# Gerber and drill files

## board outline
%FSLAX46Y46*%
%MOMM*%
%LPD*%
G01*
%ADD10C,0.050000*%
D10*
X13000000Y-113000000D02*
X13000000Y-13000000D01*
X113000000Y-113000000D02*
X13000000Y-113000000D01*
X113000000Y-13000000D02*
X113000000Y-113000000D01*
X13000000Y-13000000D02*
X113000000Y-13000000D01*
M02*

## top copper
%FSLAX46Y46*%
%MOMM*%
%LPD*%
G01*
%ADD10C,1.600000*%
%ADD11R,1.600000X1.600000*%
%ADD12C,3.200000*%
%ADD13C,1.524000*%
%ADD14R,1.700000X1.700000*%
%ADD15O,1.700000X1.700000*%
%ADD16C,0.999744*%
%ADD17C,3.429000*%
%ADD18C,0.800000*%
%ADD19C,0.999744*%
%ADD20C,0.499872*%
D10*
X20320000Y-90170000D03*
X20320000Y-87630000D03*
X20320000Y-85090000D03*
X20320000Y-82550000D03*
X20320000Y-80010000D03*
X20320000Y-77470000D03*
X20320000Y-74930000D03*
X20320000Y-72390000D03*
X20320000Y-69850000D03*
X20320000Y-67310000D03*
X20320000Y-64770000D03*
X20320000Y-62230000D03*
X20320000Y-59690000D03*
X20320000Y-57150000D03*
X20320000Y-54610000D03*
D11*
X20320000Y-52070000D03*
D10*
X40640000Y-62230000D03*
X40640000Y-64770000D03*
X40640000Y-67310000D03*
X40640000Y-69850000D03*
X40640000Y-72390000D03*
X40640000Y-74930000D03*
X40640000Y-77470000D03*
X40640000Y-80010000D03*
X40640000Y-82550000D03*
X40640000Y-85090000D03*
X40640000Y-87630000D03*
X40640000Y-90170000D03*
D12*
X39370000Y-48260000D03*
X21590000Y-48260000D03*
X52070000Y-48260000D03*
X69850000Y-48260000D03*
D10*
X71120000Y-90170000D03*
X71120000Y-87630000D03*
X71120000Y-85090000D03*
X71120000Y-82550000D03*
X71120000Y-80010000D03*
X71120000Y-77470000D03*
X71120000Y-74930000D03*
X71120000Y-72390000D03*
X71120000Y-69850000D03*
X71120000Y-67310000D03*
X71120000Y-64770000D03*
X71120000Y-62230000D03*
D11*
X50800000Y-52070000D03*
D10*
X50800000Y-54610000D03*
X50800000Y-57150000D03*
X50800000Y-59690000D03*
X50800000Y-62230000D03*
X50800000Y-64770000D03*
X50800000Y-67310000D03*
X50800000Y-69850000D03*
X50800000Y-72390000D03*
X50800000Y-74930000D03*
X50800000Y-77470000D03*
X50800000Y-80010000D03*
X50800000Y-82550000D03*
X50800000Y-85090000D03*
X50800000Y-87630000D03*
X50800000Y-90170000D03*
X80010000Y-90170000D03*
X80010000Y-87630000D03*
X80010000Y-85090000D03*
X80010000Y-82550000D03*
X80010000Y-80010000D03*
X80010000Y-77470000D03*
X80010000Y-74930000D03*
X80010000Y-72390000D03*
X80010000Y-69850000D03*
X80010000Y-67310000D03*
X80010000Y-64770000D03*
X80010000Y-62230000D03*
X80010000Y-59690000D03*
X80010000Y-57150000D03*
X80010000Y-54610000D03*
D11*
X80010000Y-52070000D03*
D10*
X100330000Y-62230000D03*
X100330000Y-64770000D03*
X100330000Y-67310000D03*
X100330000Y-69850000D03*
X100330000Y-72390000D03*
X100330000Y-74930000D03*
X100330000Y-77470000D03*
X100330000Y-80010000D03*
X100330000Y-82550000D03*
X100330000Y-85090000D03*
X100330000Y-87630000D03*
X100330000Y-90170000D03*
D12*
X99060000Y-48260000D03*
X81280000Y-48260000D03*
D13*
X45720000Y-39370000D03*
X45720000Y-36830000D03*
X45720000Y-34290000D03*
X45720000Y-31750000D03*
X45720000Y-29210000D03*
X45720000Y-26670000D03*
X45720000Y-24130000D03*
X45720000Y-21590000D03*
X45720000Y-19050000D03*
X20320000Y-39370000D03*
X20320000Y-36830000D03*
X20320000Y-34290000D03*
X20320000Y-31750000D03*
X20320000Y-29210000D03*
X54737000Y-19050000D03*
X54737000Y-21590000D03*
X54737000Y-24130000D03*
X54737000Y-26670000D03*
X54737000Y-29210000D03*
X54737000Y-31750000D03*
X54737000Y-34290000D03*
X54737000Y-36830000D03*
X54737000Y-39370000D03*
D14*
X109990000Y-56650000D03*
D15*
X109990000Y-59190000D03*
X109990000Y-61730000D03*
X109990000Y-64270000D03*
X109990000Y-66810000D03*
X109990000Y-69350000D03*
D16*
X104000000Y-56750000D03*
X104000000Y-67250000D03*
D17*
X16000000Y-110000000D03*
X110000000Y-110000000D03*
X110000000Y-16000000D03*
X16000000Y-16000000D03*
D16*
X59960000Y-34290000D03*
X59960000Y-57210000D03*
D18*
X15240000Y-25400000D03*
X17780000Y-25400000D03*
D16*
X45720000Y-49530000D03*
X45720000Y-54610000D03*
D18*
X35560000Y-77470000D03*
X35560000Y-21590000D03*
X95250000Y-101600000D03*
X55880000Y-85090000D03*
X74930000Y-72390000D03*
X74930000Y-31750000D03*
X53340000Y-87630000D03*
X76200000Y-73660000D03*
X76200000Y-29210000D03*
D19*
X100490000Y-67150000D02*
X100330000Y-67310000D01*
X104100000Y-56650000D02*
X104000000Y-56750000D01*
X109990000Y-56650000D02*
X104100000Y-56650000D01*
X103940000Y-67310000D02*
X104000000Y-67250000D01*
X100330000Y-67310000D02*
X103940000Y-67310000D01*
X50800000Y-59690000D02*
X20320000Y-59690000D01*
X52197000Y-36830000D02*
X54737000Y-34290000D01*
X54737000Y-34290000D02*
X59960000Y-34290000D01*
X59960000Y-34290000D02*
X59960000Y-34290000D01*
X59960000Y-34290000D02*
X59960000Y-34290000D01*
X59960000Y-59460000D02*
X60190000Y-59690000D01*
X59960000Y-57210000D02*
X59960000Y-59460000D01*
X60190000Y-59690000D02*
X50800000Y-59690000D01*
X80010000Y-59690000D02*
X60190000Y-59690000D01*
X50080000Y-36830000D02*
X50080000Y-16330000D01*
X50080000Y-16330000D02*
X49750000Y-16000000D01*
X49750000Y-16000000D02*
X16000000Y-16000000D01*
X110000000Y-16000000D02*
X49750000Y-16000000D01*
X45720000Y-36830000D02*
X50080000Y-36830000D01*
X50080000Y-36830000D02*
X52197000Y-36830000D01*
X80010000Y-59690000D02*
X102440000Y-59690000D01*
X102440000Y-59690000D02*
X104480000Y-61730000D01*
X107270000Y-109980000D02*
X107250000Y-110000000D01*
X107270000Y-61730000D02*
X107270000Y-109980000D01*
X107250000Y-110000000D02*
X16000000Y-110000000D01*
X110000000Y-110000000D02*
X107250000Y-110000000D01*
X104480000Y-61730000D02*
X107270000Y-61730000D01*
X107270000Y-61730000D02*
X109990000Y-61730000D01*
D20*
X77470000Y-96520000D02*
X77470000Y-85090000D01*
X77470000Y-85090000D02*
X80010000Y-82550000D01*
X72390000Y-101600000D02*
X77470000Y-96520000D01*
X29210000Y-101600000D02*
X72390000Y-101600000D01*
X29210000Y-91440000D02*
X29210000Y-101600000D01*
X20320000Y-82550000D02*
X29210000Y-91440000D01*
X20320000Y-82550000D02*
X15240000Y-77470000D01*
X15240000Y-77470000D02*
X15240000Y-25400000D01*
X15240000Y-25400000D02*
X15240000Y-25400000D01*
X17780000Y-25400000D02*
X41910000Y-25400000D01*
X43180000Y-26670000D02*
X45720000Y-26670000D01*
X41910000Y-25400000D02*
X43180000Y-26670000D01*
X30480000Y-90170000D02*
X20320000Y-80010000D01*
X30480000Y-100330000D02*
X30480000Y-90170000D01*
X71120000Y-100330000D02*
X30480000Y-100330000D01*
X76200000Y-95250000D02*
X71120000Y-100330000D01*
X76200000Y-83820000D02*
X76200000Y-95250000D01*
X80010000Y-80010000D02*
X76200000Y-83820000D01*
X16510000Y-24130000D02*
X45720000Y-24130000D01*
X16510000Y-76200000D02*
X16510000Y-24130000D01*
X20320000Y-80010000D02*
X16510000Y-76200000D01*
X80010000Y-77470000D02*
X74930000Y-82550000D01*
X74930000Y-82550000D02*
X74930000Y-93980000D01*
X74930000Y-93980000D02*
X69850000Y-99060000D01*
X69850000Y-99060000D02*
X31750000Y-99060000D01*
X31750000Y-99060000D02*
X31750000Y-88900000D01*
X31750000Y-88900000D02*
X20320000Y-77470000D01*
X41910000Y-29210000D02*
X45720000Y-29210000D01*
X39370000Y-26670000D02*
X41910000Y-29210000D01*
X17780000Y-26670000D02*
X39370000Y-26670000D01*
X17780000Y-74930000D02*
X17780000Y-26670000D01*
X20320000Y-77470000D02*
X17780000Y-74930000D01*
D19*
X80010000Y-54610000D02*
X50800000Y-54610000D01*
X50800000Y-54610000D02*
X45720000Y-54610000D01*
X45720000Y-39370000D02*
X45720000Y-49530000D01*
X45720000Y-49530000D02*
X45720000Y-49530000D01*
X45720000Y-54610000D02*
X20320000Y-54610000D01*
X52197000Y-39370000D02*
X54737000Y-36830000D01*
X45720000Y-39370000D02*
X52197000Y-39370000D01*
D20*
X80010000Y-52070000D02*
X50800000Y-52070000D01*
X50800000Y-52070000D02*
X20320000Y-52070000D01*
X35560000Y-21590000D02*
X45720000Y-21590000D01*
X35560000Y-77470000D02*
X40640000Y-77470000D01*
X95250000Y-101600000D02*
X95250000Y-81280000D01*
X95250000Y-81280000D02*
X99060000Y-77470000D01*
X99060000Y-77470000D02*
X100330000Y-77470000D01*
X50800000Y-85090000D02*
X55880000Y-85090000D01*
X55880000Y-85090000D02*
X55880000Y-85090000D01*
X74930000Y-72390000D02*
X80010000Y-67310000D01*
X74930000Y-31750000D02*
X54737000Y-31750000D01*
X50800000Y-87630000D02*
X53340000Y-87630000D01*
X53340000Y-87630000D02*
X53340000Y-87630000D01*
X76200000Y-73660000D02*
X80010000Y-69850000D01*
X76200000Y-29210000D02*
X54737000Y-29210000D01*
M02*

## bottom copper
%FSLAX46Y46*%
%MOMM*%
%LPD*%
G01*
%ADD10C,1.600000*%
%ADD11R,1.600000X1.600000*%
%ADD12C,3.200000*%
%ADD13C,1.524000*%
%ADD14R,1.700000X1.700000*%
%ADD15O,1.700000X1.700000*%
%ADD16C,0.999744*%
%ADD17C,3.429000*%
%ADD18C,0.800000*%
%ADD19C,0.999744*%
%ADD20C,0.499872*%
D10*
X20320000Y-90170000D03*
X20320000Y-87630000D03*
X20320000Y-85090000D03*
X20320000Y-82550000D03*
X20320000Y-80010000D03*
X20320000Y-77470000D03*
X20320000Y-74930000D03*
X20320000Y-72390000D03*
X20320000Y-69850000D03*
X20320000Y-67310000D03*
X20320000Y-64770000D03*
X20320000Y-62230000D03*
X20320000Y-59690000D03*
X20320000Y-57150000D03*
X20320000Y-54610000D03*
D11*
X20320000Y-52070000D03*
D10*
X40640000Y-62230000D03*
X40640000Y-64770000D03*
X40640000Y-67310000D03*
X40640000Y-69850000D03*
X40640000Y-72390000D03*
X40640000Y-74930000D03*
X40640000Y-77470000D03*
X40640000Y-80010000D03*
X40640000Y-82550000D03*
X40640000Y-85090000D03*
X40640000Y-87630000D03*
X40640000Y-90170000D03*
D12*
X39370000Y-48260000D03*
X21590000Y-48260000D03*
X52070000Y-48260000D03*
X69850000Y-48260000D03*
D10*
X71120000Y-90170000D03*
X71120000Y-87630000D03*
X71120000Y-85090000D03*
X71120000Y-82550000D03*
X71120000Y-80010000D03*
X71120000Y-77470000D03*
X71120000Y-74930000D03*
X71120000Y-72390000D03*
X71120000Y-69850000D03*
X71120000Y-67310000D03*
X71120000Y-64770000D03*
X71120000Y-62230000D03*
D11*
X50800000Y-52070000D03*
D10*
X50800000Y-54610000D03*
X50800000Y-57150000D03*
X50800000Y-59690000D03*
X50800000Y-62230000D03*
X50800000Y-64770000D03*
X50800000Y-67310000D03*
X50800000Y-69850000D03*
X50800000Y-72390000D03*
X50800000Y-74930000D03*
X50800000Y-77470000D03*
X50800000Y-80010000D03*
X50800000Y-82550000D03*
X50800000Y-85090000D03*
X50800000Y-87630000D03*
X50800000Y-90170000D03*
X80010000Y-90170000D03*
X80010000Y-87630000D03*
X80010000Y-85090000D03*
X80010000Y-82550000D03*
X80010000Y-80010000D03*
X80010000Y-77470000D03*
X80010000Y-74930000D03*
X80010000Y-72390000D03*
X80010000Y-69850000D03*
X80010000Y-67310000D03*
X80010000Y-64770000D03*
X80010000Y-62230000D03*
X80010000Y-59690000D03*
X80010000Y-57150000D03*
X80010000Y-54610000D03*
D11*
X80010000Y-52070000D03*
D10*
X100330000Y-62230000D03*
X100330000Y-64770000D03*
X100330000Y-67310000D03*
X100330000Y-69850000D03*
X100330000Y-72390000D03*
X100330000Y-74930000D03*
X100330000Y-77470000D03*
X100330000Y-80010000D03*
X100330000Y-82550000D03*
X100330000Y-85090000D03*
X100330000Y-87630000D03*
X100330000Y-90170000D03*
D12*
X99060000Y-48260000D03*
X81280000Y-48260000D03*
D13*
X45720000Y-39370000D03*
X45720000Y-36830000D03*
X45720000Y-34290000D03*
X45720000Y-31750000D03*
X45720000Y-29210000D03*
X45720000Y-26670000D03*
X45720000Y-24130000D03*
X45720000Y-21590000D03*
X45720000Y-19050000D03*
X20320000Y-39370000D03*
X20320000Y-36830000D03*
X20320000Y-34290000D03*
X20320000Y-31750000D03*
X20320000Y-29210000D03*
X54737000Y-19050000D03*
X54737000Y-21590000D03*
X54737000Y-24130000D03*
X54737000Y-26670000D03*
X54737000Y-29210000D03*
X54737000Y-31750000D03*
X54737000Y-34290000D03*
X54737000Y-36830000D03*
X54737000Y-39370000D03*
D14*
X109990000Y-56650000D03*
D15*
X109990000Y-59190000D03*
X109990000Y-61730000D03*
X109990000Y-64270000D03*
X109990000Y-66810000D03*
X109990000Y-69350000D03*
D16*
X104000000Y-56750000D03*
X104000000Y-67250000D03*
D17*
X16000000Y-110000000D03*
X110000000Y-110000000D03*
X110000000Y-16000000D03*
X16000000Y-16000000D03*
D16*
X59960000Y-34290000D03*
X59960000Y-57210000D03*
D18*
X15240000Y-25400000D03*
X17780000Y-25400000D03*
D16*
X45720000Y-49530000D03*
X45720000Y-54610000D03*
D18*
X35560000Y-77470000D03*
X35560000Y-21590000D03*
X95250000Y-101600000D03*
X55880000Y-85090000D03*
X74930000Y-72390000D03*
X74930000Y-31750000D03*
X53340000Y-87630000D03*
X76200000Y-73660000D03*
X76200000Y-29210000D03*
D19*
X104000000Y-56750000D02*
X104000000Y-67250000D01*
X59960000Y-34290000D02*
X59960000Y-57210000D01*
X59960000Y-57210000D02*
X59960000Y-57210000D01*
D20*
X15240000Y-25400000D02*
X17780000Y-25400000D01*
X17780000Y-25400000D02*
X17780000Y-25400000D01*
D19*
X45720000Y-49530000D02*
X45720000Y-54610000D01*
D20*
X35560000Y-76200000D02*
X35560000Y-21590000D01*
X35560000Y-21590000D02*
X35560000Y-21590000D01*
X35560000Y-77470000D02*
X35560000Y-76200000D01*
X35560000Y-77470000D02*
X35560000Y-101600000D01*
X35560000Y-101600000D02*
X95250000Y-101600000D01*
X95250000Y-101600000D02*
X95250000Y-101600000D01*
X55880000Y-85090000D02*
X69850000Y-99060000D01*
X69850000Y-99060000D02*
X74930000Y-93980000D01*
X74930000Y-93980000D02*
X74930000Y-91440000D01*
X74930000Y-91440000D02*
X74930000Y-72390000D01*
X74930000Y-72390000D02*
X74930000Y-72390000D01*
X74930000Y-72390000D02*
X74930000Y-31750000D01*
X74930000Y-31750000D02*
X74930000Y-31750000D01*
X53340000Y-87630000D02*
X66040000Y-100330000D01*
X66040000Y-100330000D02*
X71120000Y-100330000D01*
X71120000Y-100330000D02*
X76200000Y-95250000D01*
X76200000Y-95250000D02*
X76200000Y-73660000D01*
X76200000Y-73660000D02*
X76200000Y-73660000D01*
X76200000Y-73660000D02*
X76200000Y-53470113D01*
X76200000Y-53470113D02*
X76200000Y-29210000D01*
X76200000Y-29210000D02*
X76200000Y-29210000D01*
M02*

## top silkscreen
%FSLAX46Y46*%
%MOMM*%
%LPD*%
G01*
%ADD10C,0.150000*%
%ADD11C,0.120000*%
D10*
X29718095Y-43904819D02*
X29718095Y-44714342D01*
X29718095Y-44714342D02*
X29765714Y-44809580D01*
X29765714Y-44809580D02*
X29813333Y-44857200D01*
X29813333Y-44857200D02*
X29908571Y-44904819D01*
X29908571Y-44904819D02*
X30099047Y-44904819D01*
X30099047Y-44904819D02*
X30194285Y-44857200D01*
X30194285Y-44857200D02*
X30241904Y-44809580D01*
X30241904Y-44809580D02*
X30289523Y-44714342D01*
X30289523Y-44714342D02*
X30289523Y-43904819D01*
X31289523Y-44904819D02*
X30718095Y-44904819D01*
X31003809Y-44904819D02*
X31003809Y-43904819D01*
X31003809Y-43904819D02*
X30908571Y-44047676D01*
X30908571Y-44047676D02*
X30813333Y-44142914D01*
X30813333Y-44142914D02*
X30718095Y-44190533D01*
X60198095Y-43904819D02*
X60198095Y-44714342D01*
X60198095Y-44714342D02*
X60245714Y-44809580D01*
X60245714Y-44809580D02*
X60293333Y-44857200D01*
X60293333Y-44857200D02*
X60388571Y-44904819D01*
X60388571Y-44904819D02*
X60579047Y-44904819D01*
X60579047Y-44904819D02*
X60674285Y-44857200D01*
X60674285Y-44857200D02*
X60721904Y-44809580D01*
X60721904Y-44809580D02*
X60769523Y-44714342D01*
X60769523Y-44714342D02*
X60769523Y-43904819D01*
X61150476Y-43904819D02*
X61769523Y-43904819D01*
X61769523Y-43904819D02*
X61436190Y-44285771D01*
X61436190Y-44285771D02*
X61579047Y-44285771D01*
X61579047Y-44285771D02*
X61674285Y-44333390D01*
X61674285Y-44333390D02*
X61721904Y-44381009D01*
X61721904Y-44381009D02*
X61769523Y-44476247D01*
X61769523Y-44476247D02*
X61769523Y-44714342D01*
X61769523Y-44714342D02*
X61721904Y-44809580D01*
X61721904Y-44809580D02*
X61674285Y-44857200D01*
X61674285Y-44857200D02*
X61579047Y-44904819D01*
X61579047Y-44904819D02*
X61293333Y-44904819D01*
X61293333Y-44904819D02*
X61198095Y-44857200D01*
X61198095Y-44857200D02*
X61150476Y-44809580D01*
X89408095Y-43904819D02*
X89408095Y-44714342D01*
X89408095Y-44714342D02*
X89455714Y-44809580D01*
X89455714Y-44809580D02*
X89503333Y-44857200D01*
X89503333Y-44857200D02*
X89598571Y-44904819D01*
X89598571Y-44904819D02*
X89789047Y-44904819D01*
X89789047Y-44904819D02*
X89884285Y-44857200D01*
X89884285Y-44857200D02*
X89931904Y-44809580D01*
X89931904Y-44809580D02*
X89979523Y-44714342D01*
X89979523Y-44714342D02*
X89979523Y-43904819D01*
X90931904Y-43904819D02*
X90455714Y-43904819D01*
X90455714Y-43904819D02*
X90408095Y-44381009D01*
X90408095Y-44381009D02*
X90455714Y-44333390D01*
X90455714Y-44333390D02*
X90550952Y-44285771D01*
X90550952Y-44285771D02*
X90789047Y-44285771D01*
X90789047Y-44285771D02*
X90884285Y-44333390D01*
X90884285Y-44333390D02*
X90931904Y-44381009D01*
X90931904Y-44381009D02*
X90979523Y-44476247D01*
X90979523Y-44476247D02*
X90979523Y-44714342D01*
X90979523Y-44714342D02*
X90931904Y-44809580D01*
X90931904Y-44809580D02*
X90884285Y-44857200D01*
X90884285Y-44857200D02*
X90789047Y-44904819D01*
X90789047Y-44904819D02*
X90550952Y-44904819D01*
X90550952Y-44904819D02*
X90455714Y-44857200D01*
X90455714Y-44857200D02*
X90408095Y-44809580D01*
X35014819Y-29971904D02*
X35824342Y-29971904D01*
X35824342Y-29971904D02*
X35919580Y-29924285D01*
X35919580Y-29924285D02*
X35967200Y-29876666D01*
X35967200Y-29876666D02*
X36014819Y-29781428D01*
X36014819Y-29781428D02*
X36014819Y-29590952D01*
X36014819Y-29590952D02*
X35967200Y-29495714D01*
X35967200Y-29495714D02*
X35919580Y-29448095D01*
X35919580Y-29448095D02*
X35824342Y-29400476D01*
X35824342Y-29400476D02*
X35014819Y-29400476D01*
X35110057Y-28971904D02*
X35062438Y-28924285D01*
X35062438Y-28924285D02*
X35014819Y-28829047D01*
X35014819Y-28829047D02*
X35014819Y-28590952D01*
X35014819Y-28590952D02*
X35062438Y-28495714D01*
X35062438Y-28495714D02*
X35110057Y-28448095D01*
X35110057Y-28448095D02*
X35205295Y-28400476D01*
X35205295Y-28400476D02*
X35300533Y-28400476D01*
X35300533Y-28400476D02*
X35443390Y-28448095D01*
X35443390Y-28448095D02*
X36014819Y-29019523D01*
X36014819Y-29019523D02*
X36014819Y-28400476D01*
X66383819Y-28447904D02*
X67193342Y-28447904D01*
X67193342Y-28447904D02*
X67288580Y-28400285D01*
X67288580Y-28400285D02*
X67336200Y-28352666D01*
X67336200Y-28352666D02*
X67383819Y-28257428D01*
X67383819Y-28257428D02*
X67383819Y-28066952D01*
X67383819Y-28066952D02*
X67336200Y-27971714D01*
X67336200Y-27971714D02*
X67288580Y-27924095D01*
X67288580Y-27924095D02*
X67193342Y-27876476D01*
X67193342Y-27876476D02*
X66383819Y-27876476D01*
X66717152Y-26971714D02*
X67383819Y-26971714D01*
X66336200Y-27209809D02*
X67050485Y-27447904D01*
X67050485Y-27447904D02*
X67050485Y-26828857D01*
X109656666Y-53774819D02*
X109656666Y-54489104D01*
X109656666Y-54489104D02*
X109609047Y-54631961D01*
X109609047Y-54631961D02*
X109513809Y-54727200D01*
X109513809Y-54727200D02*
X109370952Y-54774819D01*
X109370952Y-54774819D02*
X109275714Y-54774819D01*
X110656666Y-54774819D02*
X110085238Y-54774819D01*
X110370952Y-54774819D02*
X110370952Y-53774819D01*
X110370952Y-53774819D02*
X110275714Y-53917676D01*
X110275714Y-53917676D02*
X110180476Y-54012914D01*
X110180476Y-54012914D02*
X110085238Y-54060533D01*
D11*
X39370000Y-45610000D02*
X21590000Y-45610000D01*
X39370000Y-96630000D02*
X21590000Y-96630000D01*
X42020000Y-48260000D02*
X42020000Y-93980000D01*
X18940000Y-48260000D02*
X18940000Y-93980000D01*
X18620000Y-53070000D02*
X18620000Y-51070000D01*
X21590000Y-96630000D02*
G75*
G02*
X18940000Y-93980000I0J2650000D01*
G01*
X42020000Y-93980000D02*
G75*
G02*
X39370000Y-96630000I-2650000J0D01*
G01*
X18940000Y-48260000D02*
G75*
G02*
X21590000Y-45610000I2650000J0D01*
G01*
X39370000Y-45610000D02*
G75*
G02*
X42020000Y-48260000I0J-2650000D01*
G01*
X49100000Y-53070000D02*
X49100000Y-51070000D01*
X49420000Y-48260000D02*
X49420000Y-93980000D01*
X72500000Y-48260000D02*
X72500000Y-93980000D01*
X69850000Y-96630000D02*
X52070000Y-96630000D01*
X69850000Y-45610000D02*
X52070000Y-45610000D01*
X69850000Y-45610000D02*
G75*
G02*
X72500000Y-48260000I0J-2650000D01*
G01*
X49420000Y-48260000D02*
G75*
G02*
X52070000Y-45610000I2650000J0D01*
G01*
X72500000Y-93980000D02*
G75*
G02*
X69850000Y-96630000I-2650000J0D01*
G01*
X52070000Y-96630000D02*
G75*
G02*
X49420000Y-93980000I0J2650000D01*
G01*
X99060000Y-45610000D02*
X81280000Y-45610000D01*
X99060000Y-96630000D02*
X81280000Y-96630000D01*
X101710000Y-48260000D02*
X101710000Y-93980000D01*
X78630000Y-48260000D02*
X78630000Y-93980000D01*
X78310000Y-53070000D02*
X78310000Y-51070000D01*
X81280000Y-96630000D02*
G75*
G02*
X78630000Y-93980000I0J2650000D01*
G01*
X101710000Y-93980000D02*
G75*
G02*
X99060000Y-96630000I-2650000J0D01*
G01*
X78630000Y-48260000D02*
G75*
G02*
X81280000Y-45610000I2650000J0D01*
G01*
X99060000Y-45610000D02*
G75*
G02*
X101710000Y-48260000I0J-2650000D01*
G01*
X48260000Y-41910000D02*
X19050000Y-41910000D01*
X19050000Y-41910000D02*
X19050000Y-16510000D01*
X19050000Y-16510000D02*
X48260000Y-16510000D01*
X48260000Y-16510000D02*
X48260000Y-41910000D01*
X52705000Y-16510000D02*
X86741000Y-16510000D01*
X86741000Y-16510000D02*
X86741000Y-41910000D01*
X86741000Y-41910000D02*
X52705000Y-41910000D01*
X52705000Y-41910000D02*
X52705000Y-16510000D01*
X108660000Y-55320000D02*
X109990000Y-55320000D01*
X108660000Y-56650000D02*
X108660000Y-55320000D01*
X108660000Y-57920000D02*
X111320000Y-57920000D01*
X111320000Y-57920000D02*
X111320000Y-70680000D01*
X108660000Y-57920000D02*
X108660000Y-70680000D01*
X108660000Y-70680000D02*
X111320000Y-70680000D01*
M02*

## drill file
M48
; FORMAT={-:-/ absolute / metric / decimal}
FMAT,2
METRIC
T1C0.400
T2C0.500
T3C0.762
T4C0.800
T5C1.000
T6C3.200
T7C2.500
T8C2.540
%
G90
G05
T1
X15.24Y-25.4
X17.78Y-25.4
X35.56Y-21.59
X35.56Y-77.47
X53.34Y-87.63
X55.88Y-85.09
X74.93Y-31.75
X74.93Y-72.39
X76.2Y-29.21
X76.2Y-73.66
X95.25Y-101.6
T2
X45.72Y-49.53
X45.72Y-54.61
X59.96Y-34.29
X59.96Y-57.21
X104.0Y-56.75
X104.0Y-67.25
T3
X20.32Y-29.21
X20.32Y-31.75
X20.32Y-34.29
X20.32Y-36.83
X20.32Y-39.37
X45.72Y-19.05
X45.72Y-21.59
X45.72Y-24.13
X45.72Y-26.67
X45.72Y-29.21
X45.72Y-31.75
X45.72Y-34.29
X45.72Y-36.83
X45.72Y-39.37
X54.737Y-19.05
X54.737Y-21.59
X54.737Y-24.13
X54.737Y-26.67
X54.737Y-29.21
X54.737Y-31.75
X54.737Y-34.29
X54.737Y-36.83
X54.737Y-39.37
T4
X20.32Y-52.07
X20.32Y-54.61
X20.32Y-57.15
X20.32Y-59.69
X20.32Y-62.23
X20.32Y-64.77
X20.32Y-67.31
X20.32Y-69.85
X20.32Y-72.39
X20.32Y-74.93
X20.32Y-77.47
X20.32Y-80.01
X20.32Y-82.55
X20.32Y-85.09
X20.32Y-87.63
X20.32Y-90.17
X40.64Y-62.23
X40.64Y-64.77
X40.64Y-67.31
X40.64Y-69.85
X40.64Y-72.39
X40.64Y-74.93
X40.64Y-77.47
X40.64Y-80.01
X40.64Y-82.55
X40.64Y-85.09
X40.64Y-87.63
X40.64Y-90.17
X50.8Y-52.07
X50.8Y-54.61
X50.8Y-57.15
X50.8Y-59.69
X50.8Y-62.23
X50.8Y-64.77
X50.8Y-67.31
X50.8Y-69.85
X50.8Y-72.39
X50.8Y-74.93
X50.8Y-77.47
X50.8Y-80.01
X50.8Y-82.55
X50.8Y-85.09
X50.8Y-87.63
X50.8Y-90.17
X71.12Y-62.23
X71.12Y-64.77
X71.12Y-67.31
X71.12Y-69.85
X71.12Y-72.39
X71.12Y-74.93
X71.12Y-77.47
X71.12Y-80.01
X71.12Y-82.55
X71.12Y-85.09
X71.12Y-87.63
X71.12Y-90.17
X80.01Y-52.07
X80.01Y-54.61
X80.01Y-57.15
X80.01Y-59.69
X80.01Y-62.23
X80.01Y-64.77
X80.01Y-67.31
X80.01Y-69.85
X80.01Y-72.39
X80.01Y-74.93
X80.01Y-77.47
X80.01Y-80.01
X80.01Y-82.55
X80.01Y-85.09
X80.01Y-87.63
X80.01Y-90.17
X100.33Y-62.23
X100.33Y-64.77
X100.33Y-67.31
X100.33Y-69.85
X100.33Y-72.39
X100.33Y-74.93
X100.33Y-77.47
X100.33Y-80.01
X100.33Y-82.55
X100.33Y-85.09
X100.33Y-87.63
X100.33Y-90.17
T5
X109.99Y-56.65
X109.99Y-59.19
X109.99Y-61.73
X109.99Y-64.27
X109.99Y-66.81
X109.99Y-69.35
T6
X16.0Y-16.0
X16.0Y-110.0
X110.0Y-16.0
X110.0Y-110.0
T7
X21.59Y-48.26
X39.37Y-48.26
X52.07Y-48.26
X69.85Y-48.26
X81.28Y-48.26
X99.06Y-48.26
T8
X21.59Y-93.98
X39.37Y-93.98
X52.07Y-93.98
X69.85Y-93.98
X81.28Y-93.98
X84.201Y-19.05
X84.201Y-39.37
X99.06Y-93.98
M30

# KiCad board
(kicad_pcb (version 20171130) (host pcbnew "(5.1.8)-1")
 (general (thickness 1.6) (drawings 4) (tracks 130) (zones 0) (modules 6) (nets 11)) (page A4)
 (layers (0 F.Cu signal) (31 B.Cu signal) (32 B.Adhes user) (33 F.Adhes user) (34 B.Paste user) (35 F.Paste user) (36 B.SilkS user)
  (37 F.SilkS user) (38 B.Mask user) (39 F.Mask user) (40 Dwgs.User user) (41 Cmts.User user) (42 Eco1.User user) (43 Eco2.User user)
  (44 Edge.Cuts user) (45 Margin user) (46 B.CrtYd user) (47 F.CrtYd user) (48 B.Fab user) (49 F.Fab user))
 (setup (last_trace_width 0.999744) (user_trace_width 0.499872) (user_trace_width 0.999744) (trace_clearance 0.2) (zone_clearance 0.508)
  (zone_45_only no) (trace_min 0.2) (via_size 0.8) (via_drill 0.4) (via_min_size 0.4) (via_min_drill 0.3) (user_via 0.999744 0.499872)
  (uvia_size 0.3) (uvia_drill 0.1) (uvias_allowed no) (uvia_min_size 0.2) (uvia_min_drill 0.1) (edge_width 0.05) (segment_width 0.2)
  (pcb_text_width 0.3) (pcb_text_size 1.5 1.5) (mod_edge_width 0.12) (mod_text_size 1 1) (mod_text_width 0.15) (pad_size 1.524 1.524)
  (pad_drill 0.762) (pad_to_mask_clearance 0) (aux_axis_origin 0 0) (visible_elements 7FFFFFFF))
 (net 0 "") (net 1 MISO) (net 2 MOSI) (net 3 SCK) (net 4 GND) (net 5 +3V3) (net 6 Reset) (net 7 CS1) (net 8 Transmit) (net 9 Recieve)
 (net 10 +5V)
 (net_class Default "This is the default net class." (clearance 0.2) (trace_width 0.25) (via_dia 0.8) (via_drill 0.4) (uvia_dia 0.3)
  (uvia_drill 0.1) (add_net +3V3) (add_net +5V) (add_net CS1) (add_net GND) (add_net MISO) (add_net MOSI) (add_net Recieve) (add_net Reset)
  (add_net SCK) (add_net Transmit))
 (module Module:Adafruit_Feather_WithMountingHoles (layer F.Cu) (at 20.32 52.07)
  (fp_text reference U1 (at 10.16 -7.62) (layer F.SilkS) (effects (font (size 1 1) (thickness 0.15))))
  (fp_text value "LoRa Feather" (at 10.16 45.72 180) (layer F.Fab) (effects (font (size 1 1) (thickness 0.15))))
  (fp_line (start 19.05 -6.46) (end 1.27 -6.46) (layer F.SilkS) (width 0.12))
  (fp_line (start 19.05 44.56) (end 1.27 44.56) (layer F.SilkS) (width 0.12))
  (fp_line (start 21.7 -3.81) (end 21.7 41.91) (layer F.SilkS) (width 0.12))
  (fp_line (start -1.38 -3.81) (end -1.38 41.91) (layer F.SilkS) (width 0.12))
  (fp_line (start -1.7 1) (end -1.7 -1) (layer F.SilkS) (width 0.12))
  (fp_arc (start 1.27 41.91) (end -1.38 41.91) (angle -90) (layer F.SilkS) (width 0.12))
  (fp_arc (start 19.05 41.91) (end 19.05 44.56) (angle -90) (layer F.SilkS) (width 0.12))
  (fp_arc (start 1.27 -3.81) (end 1.27 -6.46) (angle -90) (layer F.SilkS) (width 0.12))
  (fp_arc (start 19.05 -3.81) (end 21.7 -3.81) (angle -90) (layer F.SilkS) (width 0.12))
  (pad 16 thru_hole circle (at 0 38.1 180) (size 1.6 1.6) (drill 0.8) (layers *.Cu *.Mask))
  (pad 15 thru_hole circle (at 0 35.56 180) (size 1.6 1.6) (drill 0.8) (layers *.Cu *.Mask))
  (pad 14 thru_hole circle (at 0 33.02 180) (size 1.6 1.6) (drill 0.8) (layers *.Cu *.Mask))
  (pad 13 thru_hole circle (at 0 30.48 180) (size 1.6 1.6) (drill 0.8) (layers *.Cu *.Mask) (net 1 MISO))
  (pad 12 thru_hole circle (at 0 27.94 180) (size 1.6 1.6) (drill 0.8) (layers *.Cu *.Mask) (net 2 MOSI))
  (pad 11 thru_hole circle (at 0 25.4 180) (size 1.6 1.6) (drill 0.8) (layers *.Cu *.Mask) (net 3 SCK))
  (pad 10 thru_hole circle (at 0 22.86 180) (size 1.6 1.6) (drill 0.8) (layers *.Cu *.Mask))
  (pad 9 thru_hole circle (at 0 20.32 180) (size 1.6 1.6) (drill 0.8) (layers *.Cu *.Mask))
  (pad 8 thru_hole circle (at 0 17.78 180) (size 1.6 1.6) (drill 0.8) (layers *.Cu *.Mask))
  (pad 7 thru_hole circle (at 0 15.24 180) (size 1.6 1.6) (drill 0.8) (layers *.Cu *.Mask))
  (pad 6 thru_hole circle (at 0 12.7 180) (size 1.6 1.6) (drill 0.8) (layers *.Cu *.Mask))
  (pad 5 thru_hole circle (at 0 10.16 180) (size 1.6 1.6) (drill 0.8) (layers *.Cu *.Mask))
  (pad 4 thru_hole circle (at 0 7.62 180) (size 1.6 1.6) (drill 0.8) (layers *.Cu *.Mask) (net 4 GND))
  (pad 3 thru_hole circle (at 0 5.08 180) (size 1.6 1.6) (drill 0.8) (layers *.Cu *.Mask))
  (pad 2 thru_hole circle (at 0 2.54 180) (size 1.6 1.6) (drill 0.8) (layers *.Cu *.Mask) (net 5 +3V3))
  (pad 1 thru_hole rect (at 0 0 180) (size 1.6 1.6) (drill 0.8) (layers *.Cu *.Mask) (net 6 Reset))
  (pad 28 thru_hole circle (at 20.32 10.16 180) (size 1.6 1.6) (drill 0.8) (layers *.Cu *.Mask))
  (pad 27 thru_hole circle (at 20.32 12.7 180) (size 1.6 1.6) (drill 0.8) (layers *.Cu *.Mask))
  (pad 26 thru_hole circle (at 20.32 15.24 180) (size 1.6 1.6) (drill 0.8) (layers *.Cu *.Mask))
  (pad 25 thru_hole circle (at 20.32 17.78 180) (size 1.6 1.6) (drill 0.8) (layers *.Cu *.Mask))
  (pad 24 thru_hole circle (at 20.32 20.32 180) (size 1.6 1.6) (drill 0.8) (layers *.Cu *.Mask))
  (pad 23 thru_hole circle (at 20.32 22.86 180) (size 1.6 1.6) (drill 0.8) (layers *.Cu *.Mask))
  (pad 22 thru_hole circle (at 20.32 25.4 180) (size 1.6 1.6) (drill 0.8) (layers *.Cu *.Mask) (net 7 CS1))
  (pad 21 thru_hole circle (at 20.32 27.94 180) (size 1.6 1.6) (drill 0.8) (layers *.Cu *.Mask))
  (pad 20 thru_hole circle (at 20.32 30.48 180) (size 1.6 1.6) (drill 0.8) (layers *.Cu *.Mask))
  (pad 19 thru_hole circle (at 20.32 33.02 180) (size 1.6 1.6) (drill 0.8) (layers *.Cu *.Mask))
  (pad 18 thru_hole circle (at 20.32 35.56 180) (size 1.6 1.6) (drill 0.8) (layers *.Cu *.Mask))
  (pad 17 thru_hole circle (at 20.32 38.1 180) (size 1.6 1.6) (drill 0.8) (layers *.Cu *.Mask))
  (pad "" np_thru_hole circle (at 19.05 -3.81 270) (size 3.2 3.2) (drill 2.5) (layers *.Cu *.Mask))
  (pad "" np_thru_hole circle (at 19.05 41.91 270) (size 2.54 2.54) (drill 2.54) (layers *.Cu *.Mask))
  (pad "" np_thru_hole circle (at 1.27 -3.81 270) (size 3.2 3.2) (drill 2.5) (layers *.Cu *.Mask))
  (pad "" np_thru_hole circle (at 1.27 41.91 270) (size 2.54 2.54) (drill 2.54) (layers *.Cu *.Mask)))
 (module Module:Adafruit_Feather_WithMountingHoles (layer F.Cu) (at 50.8 52.07)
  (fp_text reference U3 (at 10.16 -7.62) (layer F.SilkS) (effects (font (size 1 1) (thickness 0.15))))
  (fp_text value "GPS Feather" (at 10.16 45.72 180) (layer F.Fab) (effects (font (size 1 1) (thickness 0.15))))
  (fp_line (start -1.7 1) (end -1.7 -1) (layer F.SilkS) (width 0.12))
  (fp_line (start -1.38 -3.81) (end -1.38 41.91) (layer F.SilkS) (width 0.12))
  (fp_line (start 21.7 -3.81) (end 21.7 41.91) (layer F.SilkS) (width 0.12))
  (fp_line (start 19.05 44.56) (end 1.27 44.56) (layer F.SilkS) (width 0.12))
  (fp_line (start 19.05 -6.46) (end 1.27 -6.46) (layer F.SilkS) (width 0.12))
  (fp_arc (start 19.05 -3.81) (end 21.7 -3.81) (angle -90) (layer F.SilkS) (width 0.12))
  (fp_arc (start 1.27 -3.81) (end 1.27 -6.46) (angle -90) (layer F.SilkS) (width 0.12))
  (fp_arc (start 19.05 41.91) (end 19.05 44.56) (angle -90) (layer F.SilkS) (width 0.12))
  (fp_arc (start 1.27 41.91) (end -1.38 41.91) (angle -90) (layer F.SilkS) (width 0.12))
  (pad "" np_thru_hole circle (at 1.27 41.91 270) (size 2.54 2.54) (drill 2.54) (layers *.Cu *.Mask))
  (pad "" np_thru_hole circle (at 1.27 -3.81 270) (size 3.2 3.2) (drill 2.5) (layers *.Cu *.Mask))
  (pad "" np_thru_hole circle (at 19.05 41.91 270) (size 2.54 2.54) (drill 2.54) (layers *.Cu *.Mask))
  (pad "" np_thru_hole circle (at 19.05 -3.81 270) (size 3.2 3.2) (drill 2.5) (layers *.Cu *.Mask))
  (pad 17 thru_hole circle (at 20.32 38.1 180) (size 1.6 1.6) (drill 0.8) (layers *.Cu *.Mask))
  (pad 18 thru_hole circle (at 20.32 35.56 180) (size 1.6 1.6) (drill 0.8) (layers *.Cu *.Mask))
  (pad 19 thru_hole circle (at 20.32 33.02 180) (size 1.6 1.6) (drill 0.8) (layers *.Cu *.Mask))
  (pad 20 thru_hole circle (at 20.32 30.48 180) (size 1.6 1.6) (drill 0.8) (layers *.Cu *.Mask))
  (pad 21 thru_hole circle (at 20.32 27.94 180) (size 1.6 1.6) (drill 0.8) (layers *.Cu *.Mask))
  (pad 22 thru_hole circle (at 20.32 25.4 180) (size 1.6 1.6) (drill 0.8) (layers *.Cu *.Mask))
  (pad 23 thru_hole circle (at 20.32 22.86 180) (size 1.6 1.6) (drill 0.8) (layers *.Cu *.Mask))
  (pad 24 thru_hole circle (at 20.32 20.32 180) (size 1.6 1.6) (drill 0.8) (layers *.Cu *.Mask))
  (pad 25 thru_hole circle (at 20.32 17.78 180) (size 1.6 1.6) (drill 0.8) (layers *.Cu *.Mask))
  (pad 26 thru_hole circle (at 20.32 15.24 180) (size 1.6 1.6) (drill 0.8) (layers *.Cu *.Mask))
  (pad 27 thru_hole circle (at 20.32 12.7 180) (size 1.6 1.6) (drill 0.8) (layers *.Cu *.Mask))
  (pad 28 thru_hole circle (at 20.32 10.16 180) (size 1.6 1.6) (drill 0.8) (layers *.Cu *.Mask))
  (pad 1 thru_hole rect (at 0 0 180) (size 1.6 1.6) (drill 0.8) (layers *.Cu *.Mask) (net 6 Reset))
  (pad 2 thru_hole circle (at 0 2.54 180) (size 1.6 1.6) (drill 0.8) (layers *.Cu *.Mask) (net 5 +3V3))
  (pad 3 thru_hole circle (at 0 5.08 180) (size 1.6 1.6) (drill 0.8) (layers *.Cu *.Mask))
  (pad 4 thru_hole circle (at 0 7.62 180) (size 1.6 1.6) (drill 0.8) (layers *.Cu *.Mask) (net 4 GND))
  (pad 5 thru_hole circle (at 0 10.16 180) (size 1.6 1.6) (drill 0.8) (layers *.Cu *.Mask))
  (pad 6 thru_hole circle (at 0 12.7 180) (size 1.6 1.6) (drill 0.8) (layers *.Cu *.Mask))
  (pad 7 thru_hole circle (at 0 15.24 180) (size 1.6 1.6) (drill 0.8) (layers *.Cu *.Mask))
  (pad 8 thru_hole circle (at 0 17.78 180) (size 1.6 1.6) (drill 0.8) (layers *.Cu *.Mask))
  (pad 9 thru_hole circle (at 0 20.32 180) (size 1.6 1.6) (drill 0.8) (layers *.Cu *.Mask))
  (pad 10 thru_hole circle (at 0 22.86 180) (size 1.6 1.6) (drill 0.8) (layers *.Cu *.Mask))
  (pad 11 thru_hole circle (at 0 25.4 180) (size 1.6 1.6) (drill 0.8) (layers *.Cu *.Mask))
  (pad 12 thru_hole circle (at 0 27.94 180) (size 1.6 1.6) (drill 0.8) (layers *.Cu *.Mask))
  (pad 13 thru_hole circle (at 0 30.48 180) (size 1.6 1.6) (drill 0.8) (layers *.Cu *.Mask))
  (pad 14 thru_hole circle (at 0 33.02 180) (size 1.6 1.6) (drill 0.8) (layers *.Cu *.Mask) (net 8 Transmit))
  (pad 15 thru_hole circle (at 0 35.56 180) (size 1.6 1.6) (drill 0.8) (layers *.Cu *.Mask) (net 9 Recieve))
  (pad 16 thru_hole circle (at 0 38.1 180) (size 1.6 1.6) (drill 0.8) (layers *.Cu *.Mask)))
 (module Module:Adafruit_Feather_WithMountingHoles (layer F.Cu) (at 80.01 52.07)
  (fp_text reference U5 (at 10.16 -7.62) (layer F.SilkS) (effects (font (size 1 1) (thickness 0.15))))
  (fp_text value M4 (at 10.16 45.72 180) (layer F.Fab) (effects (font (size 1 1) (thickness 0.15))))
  (fp_line (start 19.05 -6.46) (end 1.27 -6.46) (layer F.SilkS) (width 0.12))
  (fp_line (start 19.05 44.56) (end 1.27 44.56) (layer F.SilkS) (width 0.12))
  (fp_line (start 21.7 -3.81) (end 21.7 41.91) (layer F.SilkS) (width 0.12))
  (fp_line (start -1.38 -3.81) (end -1.38 41.91) (layer F.SilkS) (width 0.12))
  (fp_line (start -1.7 1) (end -1.7 -1) (layer F.SilkS) (width 0.12))
  (fp_arc (start 1.27 41.91) (end -1.38 41.91) (angle -90) (layer F.SilkS) (width 0.12))
  (fp_arc (start 19.05 41.91) (end 19.05 44.56) (angle -90) (layer F.SilkS) (width 0.12))
  (fp_arc (start 1.27 -3.81) (end 1.27 -6.46) (angle -90) (layer F.SilkS) (width 0.12))
  (fp_arc (start 19.05 -3.81) (end 21.7 -3.81) (angle -90) (layer F.SilkS) (width 0.12))
  (pad 16 thru_hole circle (at 0 38.1 180) (size 1.6 1.6) (drill 0.8) (layers *.Cu *.Mask))
  (pad 15 thru_hole circle (at 0 35.56 180) (size 1.6 1.6) (drill 0.8) (layers *.Cu *.Mask))
  (pad 14 thru_hole circle (at 0 33.02 180) (size 1.6 1.6) (drill 0.8) (layers *.Cu *.Mask))
  (pad 13 thru_hole circle (at 0 30.48 180) (size 1.6 1.6) (drill 0.8) (layers *.Cu *.Mask) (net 1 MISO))
  (pad 12 thru_hole circle (at 0 27.94 180) (size 1.6 1.6) (drill 0.8) (layers *.Cu *.Mask) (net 2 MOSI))
  (pad 11 thru_hole circle (at 0 25.4 180) (size 1.6 1.6) (drill 0.8) (layers *.Cu *.Mask) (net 3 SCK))
  (pad 10 thru_hole circle (at 0 22.86 180) (size 1.6 1.6) (drill 0.8) (layers *.Cu *.Mask))
  (pad 9 thru_hole circle (at 0 20.32 180) (size 1.6 1.6) (drill 0.8) (layers *.Cu *.Mask))
  (pad 8 thru_hole circle (at 0 17.78 180) (size 1.6 1.6) (drill 0.8) (layers *.Cu *.Mask) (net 9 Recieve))
  (pad 7 thru_hole circle (at 0 15.24 180) (size 1.6 1.6) (drill 0.8) (layers *.Cu *.Mask) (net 8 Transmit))
  (pad 6 thru_hole circle (at 0 12.7 180) (size 1.6 1.6) (drill 0.8) (layers *.Cu *.Mask))
  (pad 5 thru_hole circle (at 0 10.16 180) (size 1.6 1.6) (drill 0.8) (layers *.Cu *.Mask))
  (pad 4 thru_hole circle (at 0 7.62 180) (size 1.6 1.6) (drill 0.8) (layers *.Cu *.Mask) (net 4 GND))
  (pad 3 thru_hole circle (at 0 5.08 180) (size 1.6 1.6) (drill 0.8) (layers *.Cu *.Mask))
  (pad 2 thru_hole circle (at 0 2.54 180) (size 1.6 1.6) (drill 0.8) (layers *.Cu *.Mask) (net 5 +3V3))
  (pad 1 thru_hole rect (at 0 0 180) (size 1.6 1.6) (drill 0.8) (layers *.Cu *.Mask) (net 6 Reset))
  (pad 28 thru_hole circle (at 20.32 10.16 180) (size 1.6 1.6) (drill 0.8) (layers *.Cu *.Mask))
  (pad 27 thru_hole circle (at 20.32 12.7 180) (size 1.6 1.6) (drill 0.8) (layers *.Cu *.Mask))
  (pad 26 thru_hole circle (at 20.32 15.24 180) (size 1.6 1.6) (drill 0.8) (layers *.Cu *.Mask) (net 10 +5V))
  (pad 25 thru_hole circle (at 20.32 17.78 180) (size 1.6 1.6) (drill 0.8) (layers *.Cu *.Mask))
  (pad 24 thru_hole circle (at 20.32 20.32 180) (size 1.6 1.6) (drill 0.8) (layers *.Cu *.Mask))
  (pad 23 thru_hole circle (at 20.32 22.86 180) (size 1.6 1.6) (drill 0.8) (layers *.Cu *.Mask))
  (pad 22 thru_hole circle (at 20.32 25.4 180) (size 1.6 1.6) (drill 0.8) (layers *.Cu *.Mask) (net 7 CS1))
  (pad 21 thru_hole circle (at 20.32 27.94 180) (size 1.6 1.6) (drill 0.8) (layers *.Cu *.Mask))
  (pad 20 thru_hole circle (at 20.32 30.48 180) (size 1.6 1.6) (drill 0.8) (layers *.Cu *.Mask))
  (pad 19 thru_hole circle (at 20.32 33.02 180) (size 1.6 1.6) (drill 0.8) (layers *.Cu *.Mask))
  (pad 18 thru_hole circle (at 20.32 35.56 180) (size 1.6 1.6) (drill 0.8) (layers *.Cu *.Mask))
  (pad 17 thru_hole circle (at 20.32 38.1 180) (size 1.6 1.6) (drill 0.8) (layers *.Cu *.Mask))
  (pad "" np_thru_hole circle (at 19.05 -3.81 270) (size 3.2 3.2) (drill 2.5) (layers *.Cu *.Mask))
  (pad "" np_thru_hole circle (at 19.05 41.91 270) (size 2.54 2.54) (drill 2.54) (layers *.Cu *.Mask))
  (pad "" np_thru_hole circle (at 1.27 -3.81 270) (size 3.2 3.2) (drill 2.5) (layers *.Cu *.Mask))
  (pad "" np_thru_hole circle (at 1.27 41.91 270) (size 2.54 2.54) (drill 2.54) (layers *.Cu *.Mask)))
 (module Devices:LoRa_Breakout (layer F.Cu) (at 48.26 41.91 90)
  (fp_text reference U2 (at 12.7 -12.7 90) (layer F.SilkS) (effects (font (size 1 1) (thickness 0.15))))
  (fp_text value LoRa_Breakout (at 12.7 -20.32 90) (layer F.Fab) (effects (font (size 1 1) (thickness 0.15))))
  (fp_line (start 0 0) (end 0 -29.21) (layer F.SilkS) (width 0.12))
  (fp_line (start 0 -29.21) (end 25.4 -29.21) (layer F.SilkS) (width 0.12))
  (fp_line (start 25.4 -29.21) (end 25.4 0) (layer F.SilkS) (width 0.12))
  (fp_line (start 25.4 0) (end 0 0) (layer F.SilkS) (width 0.12))
  (pad 1 thru_hole circle (at 2.54 -2.54 90) (size 1.524 1.524) (drill 0.762) (layers *.Cu *.Mask) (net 5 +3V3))
  (pad 2 thru_hole circle (at 5.08 -2.54 90) (size 1.524 1.524) (drill 0.762) (layers *.Cu *.Mask) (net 4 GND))
  (pad 3 thru_hole circle (at 7.62 -2.54 90) (size 1.524 1.524) (drill 0.762) (layers *.Cu *.Mask))
  (pad 4 thru_hole circle (at 10.16 -2.54 90) (size 1.524 1.524) (drill 0.762) (layers *.Cu *.Mask))
  (pad 5 thru_hole circle (at 12.7 -2.54 90) (size 1.524 1.524) (drill 0.762) (layers *.Cu *.Mask) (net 3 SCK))
  (pad 6 thru_hole circle (at 15.24 -2.54 90) (size 1.524 1.524) (drill 0.762) (layers *.Cu *.Mask) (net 1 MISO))
  (pad 7 thru_hole circle (at 17.78 -2.54 90) (size 1.524 1.524) (drill 0.762) (layers *.Cu *.Mask) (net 2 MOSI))
  (pad 8 thru_hole circle (at 20.32 -2.54 90) (size 1.524 1.524) (drill 0.762) (layers *.Cu *.Mask) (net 7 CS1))
  (pad 9 thru_hole circle (at 22.86 -2.54 90) (size 1.524 1.524) (drill 0.762) (layers *.Cu *.Mask))
  (pad 10 thru_hole circle (at 2.54 -27.94 90) (size 1.524 1.524) (drill 0.762) (layers *.Cu *.Mask))
  (pad 11 thru_hole circle (at 5.08 -27.94 90) (size 1.524 1.524) (drill 0.762) (layers *.Cu *.Mask))
  (pad 12 thru_hole circle (at 7.62 -27.94 90) (size 1.524 1.524) (drill 0.762) (layers *.Cu *.Mask))
  (pad 13 thru_hole circle (at 10.16 -27.94 90) (size 1.524 1.524) (drill 0.762) (layers *.Cu *.Mask))
  (pad 14 thru_hole circle (at 12.7 -27.94 90) (size 1.524 1.524) (drill 0.762) (layers *.Cu *.Mask)))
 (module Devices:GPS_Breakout (layer F.Cu) (at 52.705 16.51 270)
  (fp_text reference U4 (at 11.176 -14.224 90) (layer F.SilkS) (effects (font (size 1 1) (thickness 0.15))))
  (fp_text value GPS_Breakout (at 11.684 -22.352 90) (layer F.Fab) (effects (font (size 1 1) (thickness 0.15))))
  (fp_line (start 0 0) (end 0 -34.036) (layer F.SilkS) (width 0.12))
  (fp_line (start 0 -34.036) (end 25.4 -34.036) (layer F.SilkS) (width 0.12))
  (fp_line (start 25.4 -34.036) (end 25.4 0) (layer F.SilkS) (width 0.12))
  (fp_line (start 25.4 0) (end 0 0) (layer F.SilkS) (width 0.12))
  (pad 1 thru_hole circle (at 2.54 -2.032 270) (size 1.524 1.524) (drill 0.762) (layers *.Cu *.Mask))
  (pad 2 thru_hole circle (at 5.08 -2.032 270) (size 1.524 1.524) (drill 0.762) (layers *.Cu *.Mask))
  (pad 3 thru_hole circle (at 7.62 -2.032 270) (size 1.524 1.524) (drill 0.762) (layers *.Cu *.Mask))
  (pad 4 thru_hole circle (at 10.16 -2.032 270) (size 1.524 1.524) (drill 0.762) (layers *.Cu *.Mask))
  (pad 5 thru_hole circle (at 12.7 -2.032 270) (size 1.524 1.524) (drill 0.762) (layers *.Cu *.Mask) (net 9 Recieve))
  (pad 6 thru_hole circle (at 15.24 -2.032 270) (size 1.524 1.524) (drill 0.762) (layers *.Cu *.Mask) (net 8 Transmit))
  (pad 7 thru_hole circle (at 17.78 -2.032 270) (size 1.524 1.524) (drill 0.762) (layers *.Cu *.Mask) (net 4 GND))
  (pad 8 thru_hole circle (at 20.32 -2.032 270) (size 1.524 1.524) (drill 0.762) (layers *.Cu *.Mask) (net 5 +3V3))
  (pad 9 thru_hole circle (at 22.86 -2.032 270) (size 1.524 1.524) (drill 0.762) (layers *.Cu *.Mask))
  (pad "" np_thru_hole circle (at 2.54 -31.496 270) (size 2.54 2.54) (drill 2.54) (layers *.Cu *.Mask))
  (pad "" np_thru_hole circle (at 22.86 -31.496 270) (size 2.54 2.54) (drill 2.54) (layers *.Cu *.Mask)))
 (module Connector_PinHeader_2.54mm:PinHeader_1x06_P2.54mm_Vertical (layer F.Cu) (at 109.99 56.65)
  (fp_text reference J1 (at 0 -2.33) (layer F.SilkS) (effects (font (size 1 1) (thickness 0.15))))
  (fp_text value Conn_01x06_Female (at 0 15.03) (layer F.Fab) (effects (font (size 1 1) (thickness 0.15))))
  (fp_line (start -1.33 -1.33) (end 0 -1.33) (layer F.SilkS) (width 0.12))
  (fp_line (start -1.33 0) (end -1.33 -1.33) (layer F.SilkS) (width 0.12))
  (fp_line (start -1.33 1.27) (end 1.33 1.27) (layer F.SilkS) (width 0.12))
  (fp_line (start 1.33 1.27) (end 1.33 14.03) (layer F.SilkS) (width 0.12))
  (fp_line (start -1.33 1.27) (end -1.33 14.03) (layer F.SilkS) (width 0.12))
  (fp_line (start -1.33 14.03) (end 1.33 14.03) (layer F.SilkS) (width 0.12))
  (pad 1 thru_hole rect (at 0 0) (size 1.7 1.7) (drill 1) (layers *.Cu *.Mask) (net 10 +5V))
  (pad 2 thru_hole oval (at 0 2.54) (size 1.7 1.7) (drill 1) (layers *.Cu *.Mask))
  (pad 3 thru_hole oval (at 0 5.08) (size 1.7 1.7) (drill 1) (layers *.Cu *.Mask) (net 4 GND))
  (pad 4 thru_hole oval (at 0 7.62) (size 1.7 1.7) (drill 1) (layers *.Cu *.Mask))
  (pad 5 thru_hole oval (at 0 10.16) (size 1.7 1.7) (drill 1) (layers *.Cu *.Mask))
  (pad 6 thru_hole oval (at 0 12.7) (size 1.7 1.7) (drill 1) (layers *.Cu *.Mask)))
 (gr_line (start 13 113) (end 13 13) (layer Edge.Cuts) (width 0.05))
 (gr_line (start 113 113) (end 13 113) (layer Edge.Cuts) (width 0.05))
 (gr_line (start 113 13) (end 113 113) (layer Edge.Cuts) (width 0.05))
 (gr_line (start 13 13) (end 113 13) (layer Edge.Cuts) (width 0.05))
 (via (at 104 56.75) (size 0.999744) (drill 0.499872) (layers F.Cu B.Cu) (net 10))
 (segment (start 104 56.75) (end 104 67.25) (width 0.999744) (layer B.Cu) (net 10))
 (via (at 104 67.25) (size 0.999744) (drill 0.499872) (layers F.Cu B.Cu) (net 10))
 (segment (start 100.49 67.15) (end 100.33 67.31) (width 0.999744) (layer F.Cu) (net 10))
 (segment (start 104.1 56.65) (end 104 56.75) (width 0.999744) (layer F.Cu) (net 10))
 (segment (start 109.99 56.65) (end 104.1 56.65) (width 0.999744) (layer F.Cu) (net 10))
 (segment (start 103.94 67.31) (end 104 67.25) (width 0.999744) (layer F.Cu) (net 10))
 (segment (start 100.33 67.31) (end 103.94 67.31) (width 0.999744) (layer F.Cu) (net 10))
 (via (at 16 110) (size 3.429) (drill 3.2004) (layers F.Cu B.Cu) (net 4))
 (segment (start 50.8 59.69) (end 20.32 59.69) (width 0.999744) (layer F.Cu) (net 4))
 (segment (start 52.197 36.83) (end 54.737 34.29) (width 0.999744) (layer F.Cu) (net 4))
 (via (at 110 110) (size 3.429) (drill 3.2004) (layers F.Cu B.Cu) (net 4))
 (via (at 110 16) (size 3.429) (drill 3.2004) (layers F.Cu B.Cu) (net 4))
 (via (at 16 16) (size 3.429) (drill 3.2004) (layers F.Cu B.Cu) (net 4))
 (segment (start 54.737 34.29) (end 59.96 34.29) (width 0.999744) (layer F.Cu) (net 4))
 (segment (start 59.96 34.29) (end 59.96 34.29) (width 0.999744) (layer F.Cu) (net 4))
 (segment (start 59.96 34.29) (end 59.96 34.29) (width 0.999744) (layer F.Cu) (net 4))
 (via (at 59.96 34.29) (size 0.999744) (drill 0.499872) (layers F.Cu B.Cu) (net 4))
 (segment (start 59.96 34.29) (end 59.96 57.21) (width 0.999744) (layer B.Cu) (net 4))
 (segment (start 59.96 57.21) (end 59.96 57.21) (width 0.999744) (layer B.Cu) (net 4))
 (via (at 59.96 57.21) (size 0.999744) (drill 0.499872) (layers F.Cu B.Cu) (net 4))
 (segment (start 59.96 59.46) (end 60.19 59.69) (width 0.999744) (layer F.Cu) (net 4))
 (segment (start 59.96 57.21) (end 59.96 59.46) (width 0.999744) (layer F.Cu) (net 4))
 (segment (start 60.19 59.69) (end 50.8 59.69) (width 0.999744) (layer F.Cu) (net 4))
 (segment (start 80.01 59.69) (end 60.19 59.69) (width 0.999744) (layer F.Cu) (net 4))
 (segment (start 50.08 36.83) (end 50.08 16.33) (width 0.999744) (layer F.Cu) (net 4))
 (segment (start 50.08 16.33) (end 49.75 16) (width 0.999744) (layer F.Cu) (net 4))
 (segment (start 49.75 16) (end 16 16) (width 0.999744) (layer F.Cu) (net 4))
 (segment (start 110 16) (end 49.75 16) (width 0.999744) (layer F.Cu) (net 4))
 (segment (start 45.72 36.83) (end 50.08 36.83) (width 0.999744) (layer F.Cu) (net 4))
 (segment (start 50.08 36.83) (end 52.197 36.83) (width 0.999744) (layer F.Cu) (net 4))
 (segment (start 80.01 59.69) (end 102.44 59.69) (width 0.999744) (layer F.Cu) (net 4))
 (segment (start 102.44 59.69) (end 104.48 61.73) (width 0.999744) (layer F.Cu) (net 4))
 (segment (start 107.27 109.98) (end 107.25 110) (width 0.999744) (layer F.Cu) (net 4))
 (segment (start 107.27 61.73) (end 107.27 109.98) (width 0.999744) (layer F.Cu) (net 4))
 (segment (start 107.25 110) (end 16 110) (width 0.999744) (layer F.Cu) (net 4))
 (segment (start 110 110) (end 107.25 110) (width 0.999744) (layer F.Cu) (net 4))
 (segment (start 104.48 61.73) (end 107.27 61.73) (width 0.999744) (layer F.Cu) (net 4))
 (segment (start 107.27 61.73) (end 109.99 61.73) (width 0.999744) (layer F.Cu) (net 4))
 (segment (start 77.47 96.52) (end 77.47 85.09) (width 0.499872) (layer F.Cu) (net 1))
 (segment (start 77.47 85.09) (end 80.01 82.55) (width 0.499872) (layer F.Cu) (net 1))
 (segment (start 72.39 101.6) (end 77.47 96.52) (width 0.499872) (layer F.Cu) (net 1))
 (segment (start 29.21 101.6) (end 72.39 101.6) (width 0.499872) (layer F.Cu) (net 1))
 (segment (start 29.21 91.44) (end 29.21 101.6) (width 0.499872) (layer F.Cu) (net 1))
 (segment (start 20.32 82.55) (end 29.21 91.44) (width 0.499872) (layer F.Cu) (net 1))
 (segment (start 20.32 82.55) (end 15.24 77.47) (width 0.499872) (layer F.Cu) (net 1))
 (segment (start 15.24 77.47) (end 15.24 25.4) (width 0.499872) (layer F.Cu) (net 1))
 (segment (start 15.24 25.4) (end 15.24 25.4) (width 0.499872) (layer F.Cu) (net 1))
 (via (at 15.24 25.4) (size 0.8) (drill 0.4) (layers F.Cu B.Cu) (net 1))
 (segment (start 15.24 25.4) (end 17.78 25.4) (width 0.499872) (layer B.Cu) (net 1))
 (segment (start 17.78 25.4) (end 17.78 25.4) (width 0.499872) (layer B.Cu) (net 1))
 (via (at 17.78 25.4) (size 0.8) (drill 0.4) (layers F.Cu B.Cu) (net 1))
 (segment (start 17.78 25.4) (end 41.91 25.4) (width 0.499872) (layer F.Cu) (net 1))
 (segment (start 43.18 26.67) (end 45.72 26.67) (width 0.499872) (layer F.Cu) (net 1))
 (segment (start 41.91 25.4) (end 43.18 26.67) (width 0.499872) (layer F.Cu) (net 1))
 (segment (start 30.48 90.17) (end 20.32 80.01) (width 0.499872) (layer F.Cu) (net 2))
 (segment (start 30.48 100.33) (end 30.48 90.17) (width 0.499872) (layer F.Cu) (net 2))
 (segment (start 71.12 100.33) (end 30.48 100.33) (width 0.499872) (layer F.Cu) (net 2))
 (segment (start 76.2 95.25) (end 71.12 100.33) (width 0.499872) (layer F.Cu) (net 2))
 (segment (start 76.2 83.82) (end 76.2 95.25) (width 0.499872) (layer F.Cu) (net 2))
 (segment (start 80.01 80.01) (end 76.2 83.82) (width 0.499872) (layer F.Cu) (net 2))
 (segment (start 16.51 24.13) (end 45.72 24.13) (width 0.499872) (layer F.Cu) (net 2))
 (segment (start 16.51 76.2) (end 16.51 24.13) (width 0.499872) (layer F.Cu) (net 2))
 (segment (start 20.32 80.01) (end 16.51 76.2) (width 0.499872) (layer F.Cu) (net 2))
 (segment (start 80.01 77.47) (end 74.93 82.55) (width 0.499872) (layer F.Cu) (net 3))
 (segment (start 74.93 82.55) (end 74.93 93.98) (width 0.499872) (layer F.Cu) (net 3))
 (segment (start 74.93 93.98) (end 69.85 99.06) (width 0.499872) (layer F.Cu) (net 3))
 (segment (start 69.85 99.06) (end 31.75 99.06) (width 0.499872) (layer F.Cu) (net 3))
 (segment (start 31.75 99.06) (end 31.75 88.9) (width 0.499872) (layer F.Cu) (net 3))
 (segment (start 31.75 88.9) (end 20.32 77.47) (width 0.499872) (layer F.Cu) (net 3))
 (segment (start 41.91 29.21) (end 45.72 29.21) (width 0.499872) (layer F.Cu) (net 3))
 (segment (start 39.37 26.67) (end 41.91 29.21) (width 0.499872) (layer F.Cu) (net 3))
 (segment (start 17.78 26.67) (end 39.37 26.67) (width 0.499872) (layer F.Cu) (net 3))
 (segment (start 17.78 74.93) (end 17.78 26.67) (width 0.499872) (layer F.Cu) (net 3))
 (segment (start 20.32 77.47) (end 17.78 74.93) (width 0.499872) (layer F.Cu) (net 3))
 (segment (start 80.01 54.61) (end 50.8 54.61) (width 0.999744) (layer F.Cu) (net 5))
 (segment (start 50.8 54.61) (end 45.72 54.61) (width 0.999744) (layer F.Cu) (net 5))
 (segment (start 45.72 39.37) (end 45.72 49.53) (width 0.999744) (layer F.Cu) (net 5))
 (segment (start 45.72 49.53) (end 45.72 49.53) (width 0.999744) (layer F.Cu) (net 5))
 (via (at 45.72 49.53) (size 0.999744) (drill 0.499872) (layers F.Cu B.Cu) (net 5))
 (segment (start 45.72 54.61) (end 20.32 54.61) (width 0.999744) (layer F.Cu) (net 5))
 (via (at 45.72 54.61) (size 0.999744) (drill 0.499872) (layers F.Cu B.Cu) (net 5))
 (segment (start 45.72 49.53) (end 45.72 54.61) (width 0.999744) (layer B.Cu) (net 5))
 (segment (start 52.197 39.37) (end 54.737 36.83) (width 0.999744) (layer F.Cu) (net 5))
 (segment (start 45.72 39.37) (end 52.197 39.37) (width 0.999744) (layer F.Cu) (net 5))
 (segment (start 80.01 52.07) (end 50.8 52.07) (width 0.499872) (layer F.Cu) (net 6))
 (segment (start 50.8 52.07) (end 20.32 52.07) (width 0.499872) (layer F.Cu) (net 6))
 (via (at 35.56 77.47) (size 0.8) (drill 0.4) (layers F.Cu B.Cu) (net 7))
 (segment (start 35.56 76.2) (end 35.56 21.59) (width 0.499872) (layer B.Cu) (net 7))
 (segment (start 35.56 21.59) (end 35.56 21.59) (width 0.499872) (layer B.Cu) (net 7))
 (via (at 35.56 21.59) (size 0.8) (drill 0.4) (layers F.Cu B.Cu) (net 7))
 (segment (start 35.56 21.59) (end 45.72 21.59) (width 0.499872) (layer F.Cu) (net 7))
 (segment (start 35.56 77.47) (end 35.56 76.2) (width 0.499872) (layer B.Cu) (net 7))
 (segment (start 35.56 77.47) (end 40.64 77.47) (width 0.499872) (layer F.Cu) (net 7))
 (segment (start 35.56 77.47) (end 35.56 101.6) (width 0.499872) (layer B.Cu) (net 7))
 (segment (start 35.56 101.6) (end 95.25 101.6) (width 0.499872) (layer B.Cu) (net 7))
 (segment (start 95.25 101.6) (end 95.25 101.6) (width 0.499872) (layer B.Cu) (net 7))
 (via (at 95.25 101.6) (size 0.8) (drill 0.4) (layers F.Cu B.Cu) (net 7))
 (segment (start 95.25 101.6) (end 95.25 81.28) (width 0.499872) (layer F.Cu) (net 7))
 (segment (start 95.25 81.28) (end 99.06 77.47) (width 0.499872) (layer F.Cu) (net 7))
 (segment (start 99.06 77.47) (end 100.33 77.47) (width 0.499872) (layer F.Cu) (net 7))
 (segment (start 50.8 85.09) (end 55.88 85.09) (width 0.499872) (layer F.Cu) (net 8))
 (segment (start 55.88 85.09) (end 55.88 85.09) (width 0.499872) (layer F.Cu) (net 8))
 (via (at 55.88 85.09) (size 0.8) (drill 0.4) (layers F.Cu B.Cu) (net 8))
 (segment (start 55.88 85.09) (end 69.85 99.06) (width 0.499872) (layer B.Cu) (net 8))
 (segment (start 69.85 99.06) (end 74.93 93.98) (width 0.499872) (layer B.Cu) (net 8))
 (segment (start 74.93 93.98) (end 74.93 91.44) (width 0.499872) (layer B.Cu) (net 8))
 (segment (start 74.93 91.44) (end 74.93 72.39) (width 0.499872) (layer B.Cu) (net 8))
 (segment (start 74.93 72.39) (end 74.93 72.39) (width 0.499872) (layer B.Cu) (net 8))
 (via (at 74.93 72.39) (size 0.8) (drill 0.4) (layers F.Cu B.Cu) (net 8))
 (segment (start 74.93 72.39) (end 80.01 67.31) (width 0.499872) (layer F.Cu) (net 8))
 (segment (start 74.93 72.39) (end 74.93 31.75) (width 0.499872) (layer B.Cu) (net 8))
 (segment (start 74.93 31.75) (end 74.93 31.75) (width 0.499872) (layer B.Cu) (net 8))
 (via (at 74.93 31.75) (size 0.8) (drill 0.4) (layers F.Cu B.Cu) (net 8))
 (segment (start 74.93 31.75) (end 54.737 31.75) (width 0.499872) (layer F.Cu) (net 8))
 (segment (start 50.8 87.63) (end 53.34 87.63) (width 0.499872) (layer F.Cu) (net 9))
 (segment (start 53.34 87.63) (end 53.34 87.63) (width 0.499872) (layer F.Cu) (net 9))
 (via (at 53.34 87.63) (size 0.8) (drill 0.4) (layers F.Cu B.Cu) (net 9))
 (segment (start 53.34 87.63) (end 66.04 100.33) (width 0.499872) (layer B.Cu) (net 9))
 (segment (start 66.04 100.33) (end 71.12 100.33) (width 0.499872) (layer B.Cu) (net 9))
 (segment (start 71.12 100.33) (end 76.2 95.25) (width 0.499872) (layer B.Cu) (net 9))
 (segment (start 76.2 95.25) (end 76.2 73.66) (width 0.499872) (layer B.Cu) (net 9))
 (segment (start 76.2 73.66) (end 76.2 73.66) (width 0.499872) (layer B.Cu) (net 9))
 (via (at 76.2 73.66) (size 0.8) (drill 0.4) (layers F.Cu B.Cu) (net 9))
 (segment (start 76.2 73.66) (end 80.01 69.85) (width 0.499872) (layer F.Cu) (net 9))
 (segment (start 76.2 73.66) (end 76.2 53.470113) (width 0.499872) (layer B.Cu) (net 9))
 (segment (start 76.2 53.470113) (end 76.2 29.21) (width 0.499872) (layer B.Cu) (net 9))
 (segment (start 76.2 29.21) (end 76.2 29.21) (width 0.499872) (layer B.Cu) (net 9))
 (via (at 76.2 29.21) (size 0.8) (drill 0.4) (layers F.Cu B.Cu) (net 9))
 (segment (start 76.2 29.21) (end 54.737 29.21) (width 0.499872) (layer F.Cu) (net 9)))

